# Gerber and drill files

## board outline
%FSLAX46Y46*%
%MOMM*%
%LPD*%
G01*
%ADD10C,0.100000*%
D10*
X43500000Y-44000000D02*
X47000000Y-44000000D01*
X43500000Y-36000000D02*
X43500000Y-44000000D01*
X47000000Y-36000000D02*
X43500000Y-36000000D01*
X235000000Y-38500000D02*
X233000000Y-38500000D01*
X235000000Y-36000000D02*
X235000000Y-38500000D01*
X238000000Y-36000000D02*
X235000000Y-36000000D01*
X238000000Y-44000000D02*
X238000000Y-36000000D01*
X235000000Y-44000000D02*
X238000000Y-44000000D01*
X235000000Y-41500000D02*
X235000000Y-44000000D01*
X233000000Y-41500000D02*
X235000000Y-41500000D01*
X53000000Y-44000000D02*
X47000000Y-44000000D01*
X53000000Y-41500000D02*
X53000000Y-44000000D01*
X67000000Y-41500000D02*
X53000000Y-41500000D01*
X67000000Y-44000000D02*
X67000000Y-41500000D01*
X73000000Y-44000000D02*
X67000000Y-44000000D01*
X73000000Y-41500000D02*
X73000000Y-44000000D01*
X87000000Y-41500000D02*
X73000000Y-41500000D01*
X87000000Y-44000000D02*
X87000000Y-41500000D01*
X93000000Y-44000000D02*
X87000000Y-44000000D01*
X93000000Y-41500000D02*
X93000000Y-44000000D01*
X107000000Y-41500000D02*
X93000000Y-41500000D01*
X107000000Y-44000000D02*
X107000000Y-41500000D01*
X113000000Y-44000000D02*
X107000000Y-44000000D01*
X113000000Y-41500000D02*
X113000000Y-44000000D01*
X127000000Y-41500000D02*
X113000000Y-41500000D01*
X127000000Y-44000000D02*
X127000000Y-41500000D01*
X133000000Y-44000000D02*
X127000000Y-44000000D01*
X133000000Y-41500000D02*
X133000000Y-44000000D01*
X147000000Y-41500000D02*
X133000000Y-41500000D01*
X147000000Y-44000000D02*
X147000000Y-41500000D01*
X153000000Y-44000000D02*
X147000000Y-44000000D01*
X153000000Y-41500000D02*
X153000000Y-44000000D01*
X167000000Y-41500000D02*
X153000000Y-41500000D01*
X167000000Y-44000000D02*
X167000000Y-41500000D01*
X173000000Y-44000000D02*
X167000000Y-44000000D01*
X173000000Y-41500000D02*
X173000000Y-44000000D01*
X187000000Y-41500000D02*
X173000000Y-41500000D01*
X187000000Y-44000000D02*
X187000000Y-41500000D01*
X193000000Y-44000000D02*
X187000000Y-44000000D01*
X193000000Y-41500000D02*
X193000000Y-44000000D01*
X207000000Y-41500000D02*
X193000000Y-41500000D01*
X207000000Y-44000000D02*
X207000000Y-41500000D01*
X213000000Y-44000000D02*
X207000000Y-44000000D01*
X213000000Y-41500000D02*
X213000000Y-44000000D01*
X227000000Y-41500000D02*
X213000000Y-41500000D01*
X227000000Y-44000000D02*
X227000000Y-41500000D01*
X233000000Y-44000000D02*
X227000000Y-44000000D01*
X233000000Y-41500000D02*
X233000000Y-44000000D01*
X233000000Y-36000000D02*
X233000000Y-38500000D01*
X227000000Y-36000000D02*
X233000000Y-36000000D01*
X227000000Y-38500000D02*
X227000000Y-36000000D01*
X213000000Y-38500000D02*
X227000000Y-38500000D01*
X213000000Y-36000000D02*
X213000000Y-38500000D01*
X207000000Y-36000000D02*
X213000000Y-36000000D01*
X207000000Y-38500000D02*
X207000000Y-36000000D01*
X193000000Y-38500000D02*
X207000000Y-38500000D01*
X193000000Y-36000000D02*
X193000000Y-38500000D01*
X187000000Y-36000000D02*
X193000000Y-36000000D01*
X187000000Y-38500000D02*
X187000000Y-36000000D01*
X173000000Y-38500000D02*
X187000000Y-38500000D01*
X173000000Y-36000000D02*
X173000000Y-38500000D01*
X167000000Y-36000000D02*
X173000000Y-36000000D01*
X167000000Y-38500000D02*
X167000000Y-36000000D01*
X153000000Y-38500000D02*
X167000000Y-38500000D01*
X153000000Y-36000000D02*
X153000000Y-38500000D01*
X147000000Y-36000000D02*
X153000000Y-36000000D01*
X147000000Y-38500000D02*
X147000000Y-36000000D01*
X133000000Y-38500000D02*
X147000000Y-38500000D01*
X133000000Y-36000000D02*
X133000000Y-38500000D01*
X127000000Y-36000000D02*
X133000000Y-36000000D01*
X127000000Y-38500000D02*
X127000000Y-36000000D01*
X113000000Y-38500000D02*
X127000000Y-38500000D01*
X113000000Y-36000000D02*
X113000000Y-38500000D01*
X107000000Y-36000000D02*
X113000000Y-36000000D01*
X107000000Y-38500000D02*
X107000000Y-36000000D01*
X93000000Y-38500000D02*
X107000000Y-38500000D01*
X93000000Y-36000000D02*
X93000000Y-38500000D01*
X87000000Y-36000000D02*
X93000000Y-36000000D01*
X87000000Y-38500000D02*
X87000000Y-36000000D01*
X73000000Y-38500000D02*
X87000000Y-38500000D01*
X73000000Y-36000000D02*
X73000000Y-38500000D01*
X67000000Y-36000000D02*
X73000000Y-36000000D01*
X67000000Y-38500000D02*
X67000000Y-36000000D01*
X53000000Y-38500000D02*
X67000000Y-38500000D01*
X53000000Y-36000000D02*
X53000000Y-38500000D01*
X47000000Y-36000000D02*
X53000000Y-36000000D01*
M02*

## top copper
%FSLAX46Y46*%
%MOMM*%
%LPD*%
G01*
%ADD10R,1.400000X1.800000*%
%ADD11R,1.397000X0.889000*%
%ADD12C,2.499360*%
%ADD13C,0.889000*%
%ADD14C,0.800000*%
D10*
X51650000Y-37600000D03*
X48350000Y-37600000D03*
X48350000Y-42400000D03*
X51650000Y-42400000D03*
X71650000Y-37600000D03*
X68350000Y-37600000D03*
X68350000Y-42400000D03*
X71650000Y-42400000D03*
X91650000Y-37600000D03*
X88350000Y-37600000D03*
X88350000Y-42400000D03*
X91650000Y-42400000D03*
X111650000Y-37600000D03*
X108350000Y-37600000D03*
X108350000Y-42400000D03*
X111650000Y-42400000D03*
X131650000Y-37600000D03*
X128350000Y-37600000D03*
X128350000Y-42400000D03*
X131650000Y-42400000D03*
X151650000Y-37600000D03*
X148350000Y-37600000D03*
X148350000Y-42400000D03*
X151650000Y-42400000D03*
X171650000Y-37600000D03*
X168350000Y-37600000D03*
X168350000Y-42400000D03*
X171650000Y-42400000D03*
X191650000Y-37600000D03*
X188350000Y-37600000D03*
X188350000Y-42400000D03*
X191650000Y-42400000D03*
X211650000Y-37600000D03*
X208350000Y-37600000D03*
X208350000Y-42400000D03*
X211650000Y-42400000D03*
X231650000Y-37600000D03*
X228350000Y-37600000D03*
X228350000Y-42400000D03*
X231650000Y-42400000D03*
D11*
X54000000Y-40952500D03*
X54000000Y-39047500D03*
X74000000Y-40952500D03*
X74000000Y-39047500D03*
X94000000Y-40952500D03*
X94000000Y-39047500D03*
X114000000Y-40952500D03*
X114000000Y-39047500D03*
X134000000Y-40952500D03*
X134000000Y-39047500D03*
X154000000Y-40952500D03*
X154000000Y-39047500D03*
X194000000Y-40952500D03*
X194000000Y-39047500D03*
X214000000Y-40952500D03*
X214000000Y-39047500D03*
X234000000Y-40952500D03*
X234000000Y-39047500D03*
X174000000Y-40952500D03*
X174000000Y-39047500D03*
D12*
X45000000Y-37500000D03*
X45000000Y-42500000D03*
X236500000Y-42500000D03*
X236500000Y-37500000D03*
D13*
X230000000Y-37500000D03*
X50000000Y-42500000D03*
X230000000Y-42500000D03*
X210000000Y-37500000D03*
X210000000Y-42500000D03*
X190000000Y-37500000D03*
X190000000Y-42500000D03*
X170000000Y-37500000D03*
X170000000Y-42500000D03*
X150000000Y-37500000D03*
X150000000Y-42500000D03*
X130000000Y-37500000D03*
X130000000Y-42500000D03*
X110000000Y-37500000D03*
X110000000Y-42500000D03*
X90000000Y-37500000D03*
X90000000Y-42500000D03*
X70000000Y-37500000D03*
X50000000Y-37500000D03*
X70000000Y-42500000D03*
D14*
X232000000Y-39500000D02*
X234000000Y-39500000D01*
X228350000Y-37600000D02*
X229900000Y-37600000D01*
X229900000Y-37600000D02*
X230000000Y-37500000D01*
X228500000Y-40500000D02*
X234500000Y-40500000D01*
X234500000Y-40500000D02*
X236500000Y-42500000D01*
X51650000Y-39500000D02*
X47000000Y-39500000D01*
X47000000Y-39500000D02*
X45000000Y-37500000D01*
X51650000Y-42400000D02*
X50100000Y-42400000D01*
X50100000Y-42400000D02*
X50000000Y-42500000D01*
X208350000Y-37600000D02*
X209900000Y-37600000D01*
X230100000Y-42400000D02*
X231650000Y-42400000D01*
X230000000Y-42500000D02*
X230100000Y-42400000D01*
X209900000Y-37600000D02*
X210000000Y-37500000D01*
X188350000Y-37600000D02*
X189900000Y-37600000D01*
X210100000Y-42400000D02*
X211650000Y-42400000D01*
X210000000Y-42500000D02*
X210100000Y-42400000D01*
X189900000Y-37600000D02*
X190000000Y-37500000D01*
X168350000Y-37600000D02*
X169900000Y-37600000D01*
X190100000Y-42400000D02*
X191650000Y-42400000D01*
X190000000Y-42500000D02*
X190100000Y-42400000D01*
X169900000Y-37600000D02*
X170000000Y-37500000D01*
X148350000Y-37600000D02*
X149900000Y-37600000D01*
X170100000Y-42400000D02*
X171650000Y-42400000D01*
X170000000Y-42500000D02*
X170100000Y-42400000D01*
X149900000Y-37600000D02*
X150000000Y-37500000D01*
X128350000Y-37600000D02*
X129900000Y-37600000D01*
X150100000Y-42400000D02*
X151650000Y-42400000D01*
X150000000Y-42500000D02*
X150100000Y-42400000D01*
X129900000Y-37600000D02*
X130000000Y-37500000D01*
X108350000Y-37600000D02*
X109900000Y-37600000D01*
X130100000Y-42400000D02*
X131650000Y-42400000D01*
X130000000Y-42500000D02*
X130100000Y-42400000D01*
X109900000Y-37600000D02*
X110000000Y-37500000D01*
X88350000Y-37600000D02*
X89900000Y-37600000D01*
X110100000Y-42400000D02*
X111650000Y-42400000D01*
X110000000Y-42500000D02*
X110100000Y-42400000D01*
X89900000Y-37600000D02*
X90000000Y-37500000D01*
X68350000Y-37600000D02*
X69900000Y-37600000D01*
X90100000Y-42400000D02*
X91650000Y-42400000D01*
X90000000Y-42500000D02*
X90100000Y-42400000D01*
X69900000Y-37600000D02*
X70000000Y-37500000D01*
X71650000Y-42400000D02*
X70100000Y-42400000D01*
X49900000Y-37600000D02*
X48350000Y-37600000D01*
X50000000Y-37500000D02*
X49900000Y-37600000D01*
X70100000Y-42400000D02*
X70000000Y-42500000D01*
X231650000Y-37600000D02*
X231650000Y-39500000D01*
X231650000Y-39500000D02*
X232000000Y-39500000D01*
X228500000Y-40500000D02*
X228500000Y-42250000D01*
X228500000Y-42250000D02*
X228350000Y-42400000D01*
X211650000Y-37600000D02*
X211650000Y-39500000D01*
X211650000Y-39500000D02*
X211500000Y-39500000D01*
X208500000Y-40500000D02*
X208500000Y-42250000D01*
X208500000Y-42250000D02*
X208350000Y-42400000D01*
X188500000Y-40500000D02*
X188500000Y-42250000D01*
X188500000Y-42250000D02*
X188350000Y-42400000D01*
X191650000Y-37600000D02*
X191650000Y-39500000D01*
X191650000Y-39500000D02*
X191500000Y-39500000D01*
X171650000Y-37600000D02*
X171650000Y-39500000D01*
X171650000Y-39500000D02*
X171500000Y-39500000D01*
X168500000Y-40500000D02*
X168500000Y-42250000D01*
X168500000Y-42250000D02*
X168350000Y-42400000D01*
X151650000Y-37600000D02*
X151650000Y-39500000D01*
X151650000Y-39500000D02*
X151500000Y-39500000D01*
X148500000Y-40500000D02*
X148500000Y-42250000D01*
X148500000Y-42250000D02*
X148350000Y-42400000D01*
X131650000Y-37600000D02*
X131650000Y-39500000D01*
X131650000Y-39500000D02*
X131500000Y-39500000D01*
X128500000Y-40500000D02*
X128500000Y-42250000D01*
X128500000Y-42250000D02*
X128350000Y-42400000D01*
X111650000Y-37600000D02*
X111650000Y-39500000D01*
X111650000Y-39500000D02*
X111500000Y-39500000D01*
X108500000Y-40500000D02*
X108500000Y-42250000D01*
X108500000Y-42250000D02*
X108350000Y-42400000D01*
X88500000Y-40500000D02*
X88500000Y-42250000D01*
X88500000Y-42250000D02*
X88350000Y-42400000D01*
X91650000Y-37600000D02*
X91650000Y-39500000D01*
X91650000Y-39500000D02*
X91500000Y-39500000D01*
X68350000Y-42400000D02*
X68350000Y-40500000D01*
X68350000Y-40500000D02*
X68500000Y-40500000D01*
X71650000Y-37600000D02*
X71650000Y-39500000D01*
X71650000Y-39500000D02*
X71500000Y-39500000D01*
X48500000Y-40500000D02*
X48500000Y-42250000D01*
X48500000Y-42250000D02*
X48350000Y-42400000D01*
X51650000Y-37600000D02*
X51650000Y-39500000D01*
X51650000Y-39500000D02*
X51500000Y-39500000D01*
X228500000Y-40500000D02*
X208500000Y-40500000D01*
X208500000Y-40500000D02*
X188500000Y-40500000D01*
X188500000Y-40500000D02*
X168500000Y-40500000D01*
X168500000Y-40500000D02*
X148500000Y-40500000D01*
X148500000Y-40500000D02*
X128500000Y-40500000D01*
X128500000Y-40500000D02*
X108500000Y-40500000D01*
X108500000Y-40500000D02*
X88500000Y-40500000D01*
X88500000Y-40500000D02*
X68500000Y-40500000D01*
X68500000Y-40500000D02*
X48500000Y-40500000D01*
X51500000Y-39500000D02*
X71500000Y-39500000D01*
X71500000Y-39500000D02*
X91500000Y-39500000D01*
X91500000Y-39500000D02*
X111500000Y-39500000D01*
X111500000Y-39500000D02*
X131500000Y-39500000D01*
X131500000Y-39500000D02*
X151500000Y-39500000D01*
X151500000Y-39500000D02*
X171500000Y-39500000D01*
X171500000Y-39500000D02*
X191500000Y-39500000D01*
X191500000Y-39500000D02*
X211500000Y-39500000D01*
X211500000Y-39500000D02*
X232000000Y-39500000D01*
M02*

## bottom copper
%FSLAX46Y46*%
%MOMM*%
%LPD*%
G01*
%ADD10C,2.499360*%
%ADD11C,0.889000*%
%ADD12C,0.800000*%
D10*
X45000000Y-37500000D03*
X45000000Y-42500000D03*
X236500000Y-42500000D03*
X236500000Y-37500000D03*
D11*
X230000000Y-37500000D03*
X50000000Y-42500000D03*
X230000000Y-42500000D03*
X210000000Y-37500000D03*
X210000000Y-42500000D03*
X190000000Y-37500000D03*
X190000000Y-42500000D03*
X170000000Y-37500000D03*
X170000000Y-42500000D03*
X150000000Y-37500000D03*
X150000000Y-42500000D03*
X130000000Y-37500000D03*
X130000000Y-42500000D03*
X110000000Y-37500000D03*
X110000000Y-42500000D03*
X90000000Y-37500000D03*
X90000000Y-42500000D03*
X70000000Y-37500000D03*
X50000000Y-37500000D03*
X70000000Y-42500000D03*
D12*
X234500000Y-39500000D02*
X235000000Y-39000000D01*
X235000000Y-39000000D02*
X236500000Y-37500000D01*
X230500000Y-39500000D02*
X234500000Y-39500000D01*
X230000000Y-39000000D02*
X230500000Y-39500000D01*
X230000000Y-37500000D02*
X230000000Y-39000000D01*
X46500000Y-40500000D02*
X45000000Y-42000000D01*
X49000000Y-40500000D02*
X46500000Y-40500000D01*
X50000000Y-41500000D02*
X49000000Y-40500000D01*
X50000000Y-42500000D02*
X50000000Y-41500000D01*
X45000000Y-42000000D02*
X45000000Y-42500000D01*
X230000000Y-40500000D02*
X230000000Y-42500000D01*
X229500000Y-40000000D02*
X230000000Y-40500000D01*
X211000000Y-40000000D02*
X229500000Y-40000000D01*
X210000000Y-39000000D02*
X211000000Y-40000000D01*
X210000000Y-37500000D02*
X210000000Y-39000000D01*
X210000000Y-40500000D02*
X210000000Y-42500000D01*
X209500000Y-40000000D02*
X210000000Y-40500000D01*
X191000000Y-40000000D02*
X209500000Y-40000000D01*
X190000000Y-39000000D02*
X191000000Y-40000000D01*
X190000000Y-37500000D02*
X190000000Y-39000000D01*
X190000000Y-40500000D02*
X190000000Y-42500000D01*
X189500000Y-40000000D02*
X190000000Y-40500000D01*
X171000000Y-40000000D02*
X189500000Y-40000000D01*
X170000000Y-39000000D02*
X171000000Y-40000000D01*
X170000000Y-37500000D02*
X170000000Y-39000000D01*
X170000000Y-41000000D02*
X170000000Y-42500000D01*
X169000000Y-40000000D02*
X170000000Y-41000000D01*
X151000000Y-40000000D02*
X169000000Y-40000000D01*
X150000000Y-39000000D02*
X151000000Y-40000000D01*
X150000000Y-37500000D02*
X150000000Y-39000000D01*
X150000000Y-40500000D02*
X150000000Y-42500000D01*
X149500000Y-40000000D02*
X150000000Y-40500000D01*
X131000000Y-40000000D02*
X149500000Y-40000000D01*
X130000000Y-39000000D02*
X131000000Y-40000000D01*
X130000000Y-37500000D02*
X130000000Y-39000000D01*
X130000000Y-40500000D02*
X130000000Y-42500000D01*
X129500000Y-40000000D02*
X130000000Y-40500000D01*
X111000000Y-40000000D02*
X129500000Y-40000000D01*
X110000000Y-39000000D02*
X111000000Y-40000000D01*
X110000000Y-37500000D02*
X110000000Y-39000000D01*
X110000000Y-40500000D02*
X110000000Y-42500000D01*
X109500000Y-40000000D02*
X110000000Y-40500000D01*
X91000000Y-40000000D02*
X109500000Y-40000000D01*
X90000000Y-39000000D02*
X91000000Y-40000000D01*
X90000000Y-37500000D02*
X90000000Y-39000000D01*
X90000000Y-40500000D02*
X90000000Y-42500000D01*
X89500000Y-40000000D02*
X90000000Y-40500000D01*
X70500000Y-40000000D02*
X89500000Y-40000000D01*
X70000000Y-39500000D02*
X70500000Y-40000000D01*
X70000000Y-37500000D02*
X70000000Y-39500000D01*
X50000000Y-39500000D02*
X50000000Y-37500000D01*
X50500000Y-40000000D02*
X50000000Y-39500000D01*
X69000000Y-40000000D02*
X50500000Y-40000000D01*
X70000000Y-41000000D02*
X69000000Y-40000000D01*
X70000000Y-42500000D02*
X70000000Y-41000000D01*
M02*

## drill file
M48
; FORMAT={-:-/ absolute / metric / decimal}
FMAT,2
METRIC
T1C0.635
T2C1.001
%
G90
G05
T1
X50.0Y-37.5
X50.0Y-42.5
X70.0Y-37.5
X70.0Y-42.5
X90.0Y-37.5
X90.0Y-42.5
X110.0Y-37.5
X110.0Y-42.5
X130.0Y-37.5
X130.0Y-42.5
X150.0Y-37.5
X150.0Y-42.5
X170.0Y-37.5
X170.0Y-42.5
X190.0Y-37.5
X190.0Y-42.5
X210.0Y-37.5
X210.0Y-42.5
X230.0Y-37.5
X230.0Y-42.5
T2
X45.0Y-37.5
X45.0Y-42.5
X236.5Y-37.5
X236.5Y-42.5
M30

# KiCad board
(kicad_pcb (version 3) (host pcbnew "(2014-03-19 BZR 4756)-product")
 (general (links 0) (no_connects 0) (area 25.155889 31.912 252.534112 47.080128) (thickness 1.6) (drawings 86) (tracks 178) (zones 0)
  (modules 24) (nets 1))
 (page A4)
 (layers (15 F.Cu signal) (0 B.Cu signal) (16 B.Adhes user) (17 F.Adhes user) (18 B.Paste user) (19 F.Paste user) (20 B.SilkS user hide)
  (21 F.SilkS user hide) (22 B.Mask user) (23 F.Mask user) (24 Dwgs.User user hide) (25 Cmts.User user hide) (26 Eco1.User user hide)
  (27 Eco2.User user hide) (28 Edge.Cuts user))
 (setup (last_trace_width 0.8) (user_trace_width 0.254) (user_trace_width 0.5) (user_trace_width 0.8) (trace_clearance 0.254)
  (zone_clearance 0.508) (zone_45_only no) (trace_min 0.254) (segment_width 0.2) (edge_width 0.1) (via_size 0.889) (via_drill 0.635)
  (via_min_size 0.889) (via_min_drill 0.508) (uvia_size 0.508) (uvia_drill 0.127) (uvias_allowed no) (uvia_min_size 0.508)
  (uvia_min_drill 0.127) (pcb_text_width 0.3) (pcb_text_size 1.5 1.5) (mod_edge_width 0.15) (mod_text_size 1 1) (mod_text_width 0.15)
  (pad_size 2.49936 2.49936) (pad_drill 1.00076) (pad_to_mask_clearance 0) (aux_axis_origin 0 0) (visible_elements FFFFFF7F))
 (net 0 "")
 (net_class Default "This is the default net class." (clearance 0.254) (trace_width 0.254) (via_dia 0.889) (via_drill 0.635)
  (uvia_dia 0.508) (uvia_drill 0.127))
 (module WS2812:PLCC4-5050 (layer F.Cu) (at 50 40)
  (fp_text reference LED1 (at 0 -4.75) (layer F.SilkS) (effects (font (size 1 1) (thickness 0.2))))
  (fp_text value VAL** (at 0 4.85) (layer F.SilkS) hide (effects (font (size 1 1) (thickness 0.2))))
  (pad 1 smd rect (at 1.65 -2.4) (size 1.4 1.8) (layers F.Cu F.Paste F.Mask))
  (pad 2 smd rect (at -1.65 -2.4) (size 1.4 1.8) (layers F.Cu F.Paste F.Mask))
  (pad 3 smd rect (at -1.65 2.4) (size 1.4 1.8) (layers F.Cu F.Paste F.Mask))
  (pad 4 smd rect (at 1.65 2.4) (size 1.4 1.8) (layers F.Cu F.Paste F.Mask)))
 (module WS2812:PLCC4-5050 (layer F.Cu) (at 70 40)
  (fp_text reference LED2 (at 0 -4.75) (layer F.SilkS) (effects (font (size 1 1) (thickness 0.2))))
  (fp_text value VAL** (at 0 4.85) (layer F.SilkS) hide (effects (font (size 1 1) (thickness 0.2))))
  (pad 1 smd rect (at 1.65 -2.4) (size 1.4 1.8) (layers F.Cu F.Paste F.Mask))
  (pad 2 smd rect (at -1.65 -2.4) (size 1.4 1.8) (layers F.Cu F.Paste F.Mask))
  (pad 3 smd rect (at -1.65 2.4) (size 1.4 1.8) (layers F.Cu F.Paste F.Mask))
  (pad 4 smd rect (at 1.65 2.4) (size 1.4 1.8) (layers F.Cu F.Paste F.Mask)))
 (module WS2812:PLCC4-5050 (layer F.Cu) (at 90 40)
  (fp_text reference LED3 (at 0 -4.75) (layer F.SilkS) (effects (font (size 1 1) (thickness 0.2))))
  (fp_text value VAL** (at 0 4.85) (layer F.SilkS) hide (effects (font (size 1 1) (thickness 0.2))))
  (pad 1 smd rect (at 1.65 -2.4) (size 1.4 1.8) (layers F.Cu F.Paste F.Mask))
  (pad 2 smd rect (at -1.65 -2.4) (size 1.4 1.8) (layers F.Cu F.Paste F.Mask))
  (pad 3 smd rect (at -1.65 2.4) (size 1.4 1.8) (layers F.Cu F.Paste F.Mask))
  (pad 4 smd rect (at 1.65 2.4) (size 1.4 1.8) (layers F.Cu F.Paste F.Mask)))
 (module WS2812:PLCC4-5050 (layer F.Cu) (at 110 40)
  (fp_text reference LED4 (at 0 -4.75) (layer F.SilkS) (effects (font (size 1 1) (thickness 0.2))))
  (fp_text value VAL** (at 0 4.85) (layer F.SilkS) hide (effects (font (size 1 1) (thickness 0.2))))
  (pad 1 smd rect (at 1.65 -2.4) (size 1.4 1.8) (layers F.Cu F.Paste F.Mask))
  (pad 2 smd rect (at -1.65 -2.4) (size 1.4 1.8) (layers F.Cu F.Paste F.Mask))
  (pad 3 smd rect (at -1.65 2.4) (size 1.4 1.8) (layers F.Cu F.Paste F.Mask))
  (pad 4 smd rect (at 1.65 2.4) (size 1.4 1.8) (layers F.Cu F.Paste F.Mask)))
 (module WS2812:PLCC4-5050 (layer F.Cu) (at 130 40)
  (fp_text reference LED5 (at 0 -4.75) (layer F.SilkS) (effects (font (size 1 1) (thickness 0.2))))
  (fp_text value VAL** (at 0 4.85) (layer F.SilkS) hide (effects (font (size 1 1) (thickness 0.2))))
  (pad 1 smd rect (at 1.65 -2.4) (size 1.4 1.8) (layers F.Cu F.Paste F.Mask))
  (pad 2 smd rect (at -1.65 -2.4) (size 1.4 1.8) (layers F.Cu F.Paste F.Mask))
  (pad 3 smd rect (at -1.65 2.4) (size 1.4 1.8) (layers F.Cu F.Paste F.Mask))
  (pad 4 smd rect (at 1.65 2.4) (size 1.4 1.8) (layers F.Cu F.Paste F.Mask)))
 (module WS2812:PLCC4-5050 (layer F.Cu) (at 150 40)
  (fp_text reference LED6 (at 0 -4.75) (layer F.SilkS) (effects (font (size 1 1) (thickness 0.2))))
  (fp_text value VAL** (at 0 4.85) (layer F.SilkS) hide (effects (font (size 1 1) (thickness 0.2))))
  (pad 1 smd rect (at 1.65 -2.4) (size 1.4 1.8) (layers F.Cu F.Paste F.Mask))
  (pad 2 smd rect (at -1.65 -2.4) (size 1.4 1.8) (layers F.Cu F.Paste F.Mask))
  (pad 3 smd rect (at -1.65 2.4) (size 1.4 1.8) (layers F.Cu F.Paste F.Mask))
  (pad 4 smd rect (at 1.65 2.4) (size 1.4 1.8) (layers F.Cu F.Paste F.Mask)))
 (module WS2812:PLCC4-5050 (layer F.Cu) (at 170 40)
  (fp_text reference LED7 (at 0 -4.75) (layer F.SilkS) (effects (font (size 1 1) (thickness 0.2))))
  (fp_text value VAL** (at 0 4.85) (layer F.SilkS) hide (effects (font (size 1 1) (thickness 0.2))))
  (pad 1 smd rect (at 1.65 -2.4) (size 1.4 1.8) (layers F.Cu F.Paste F.Mask))
  (pad 2 smd rect (at -1.65 -2.4) (size 1.4 1.8) (layers F.Cu F.Paste F.Mask))
  (pad 3 smd rect (at -1.65 2.4) (size 1.4 1.8) (layers F.Cu F.Paste F.Mask))
  (pad 4 smd rect (at 1.65 2.4) (size 1.4 1.8) (layers F.Cu F.Paste F.Mask)))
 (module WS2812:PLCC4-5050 (layer F.Cu) (at 190 40)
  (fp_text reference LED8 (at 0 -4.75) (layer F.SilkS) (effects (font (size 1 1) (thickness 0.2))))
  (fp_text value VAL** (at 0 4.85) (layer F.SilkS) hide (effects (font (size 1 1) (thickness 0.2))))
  (pad 1 smd rect (at 1.65 -2.4) (size 1.4 1.8) (layers F.Cu F.Paste F.Mask))
  (pad 2 smd rect (at -1.65 -2.4) (size 1.4 1.8) (layers F.Cu F.Paste F.Mask))
  (pad 3 smd rect (at -1.65 2.4) (size 1.4 1.8) (layers F.Cu F.Paste F.Mask))
  (pad 4 smd rect (at 1.65 2.4) (size 1.4 1.8) (layers F.Cu F.Paste F.Mask)))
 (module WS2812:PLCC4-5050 (layer F.Cu) (at 210 40)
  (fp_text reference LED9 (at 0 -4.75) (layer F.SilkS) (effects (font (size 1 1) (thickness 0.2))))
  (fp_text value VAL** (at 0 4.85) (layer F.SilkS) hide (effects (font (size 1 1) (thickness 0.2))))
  (pad 1 smd rect (at 1.65 -2.4) (size 1.4 1.8) (layers F.Cu F.Paste F.Mask))
  (pad 2 smd rect (at -1.65 -2.4) (size 1.4 1.8) (layers F.Cu F.Paste F.Mask))
  (pad 3 smd rect (at -1.65 2.4) (size 1.4 1.8) (layers F.Cu F.Paste F.Mask))
  (pad 4 smd rect (at 1.65 2.4) (size 1.4 1.8) (layers F.Cu F.Paste F.Mask)))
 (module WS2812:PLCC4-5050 (layer F.Cu) (at 230 40)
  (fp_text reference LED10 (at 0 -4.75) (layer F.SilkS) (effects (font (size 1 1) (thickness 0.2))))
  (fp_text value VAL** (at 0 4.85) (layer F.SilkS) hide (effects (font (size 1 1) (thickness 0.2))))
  (pad 1 smd rect (at 1.65 -2.4) (size 1.4 1.8) (layers F.Cu F.Paste F.Mask))
  (pad 2 smd rect (at -1.65 -2.4) (size 1.4 1.8) (layers F.Cu F.Paste F.Mask))
  (pad 3 smd rect (at -1.65 2.4) (size 1.4 1.8) (layers F.Cu F.Paste F.Mask))
  (pad 4 smd rect (at 1.65 2.4) (size 1.4 1.8) (layers F.Cu F.Paste F.Mask)))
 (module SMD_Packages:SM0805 (layer F.Cu) (at 54 40 90)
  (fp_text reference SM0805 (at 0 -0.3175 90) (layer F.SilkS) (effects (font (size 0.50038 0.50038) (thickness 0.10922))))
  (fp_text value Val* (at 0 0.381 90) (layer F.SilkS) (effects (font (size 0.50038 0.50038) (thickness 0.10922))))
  (pad 1 smd rect (at -0.9525 0 90) (size 0.889 1.397) (layers F.Cu F.Paste F.Mask))
  (pad 2 smd rect (at 0.9525 0 90) (size 0.889 1.397) (layers F.Cu F.Paste F.Mask)))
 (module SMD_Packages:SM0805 (layer F.Cu) (at 74 40 90)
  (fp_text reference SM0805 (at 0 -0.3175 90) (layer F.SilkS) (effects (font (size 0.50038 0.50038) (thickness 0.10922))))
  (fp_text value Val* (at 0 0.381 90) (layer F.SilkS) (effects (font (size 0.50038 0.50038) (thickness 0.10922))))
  (pad 1 smd rect (at -0.9525 0 90) (size 0.889 1.397) (layers F.Cu F.Paste F.Mask))
  (pad 2 smd rect (at 0.9525 0 90) (size 0.889 1.397) (layers F.Cu F.Paste F.Mask)))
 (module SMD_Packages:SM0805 (layer F.Cu) (at 94 40 90)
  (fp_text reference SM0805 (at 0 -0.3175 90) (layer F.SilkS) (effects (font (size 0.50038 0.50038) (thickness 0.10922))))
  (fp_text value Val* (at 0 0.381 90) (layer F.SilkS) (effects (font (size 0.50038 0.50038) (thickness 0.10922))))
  (pad 1 smd rect (at -0.9525 0 90) (size 0.889 1.397) (layers F.Cu F.Paste F.Mask))
  (pad 2 smd rect (at 0.9525 0 90) (size 0.889 1.397) (layers F.Cu F.Paste F.Mask)))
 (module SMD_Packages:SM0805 (layer F.Cu) (at 114 40 90)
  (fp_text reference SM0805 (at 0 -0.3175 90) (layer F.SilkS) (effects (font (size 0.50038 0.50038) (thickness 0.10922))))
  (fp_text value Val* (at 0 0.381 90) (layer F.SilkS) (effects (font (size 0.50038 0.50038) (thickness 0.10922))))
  (pad 1 smd rect (at -0.9525 0 90) (size 0.889 1.397) (layers F.Cu F.Paste F.Mask))
  (pad 2 smd rect (at 0.9525 0 90) (size 0.889 1.397) (layers F.Cu F.Paste F.Mask)))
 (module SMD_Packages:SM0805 (layer F.Cu) (at 134 40 90)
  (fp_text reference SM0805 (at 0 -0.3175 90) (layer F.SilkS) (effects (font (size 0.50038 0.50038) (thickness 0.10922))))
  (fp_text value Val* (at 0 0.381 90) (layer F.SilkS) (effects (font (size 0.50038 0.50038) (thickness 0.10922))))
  (pad 1 smd rect (at -0.9525 0 90) (size 0.889 1.397) (layers F.Cu F.Paste F.Mask))
  (pad 2 smd rect (at 0.9525 0 90) (size 0.889 1.397) (layers F.Cu F.Paste F.Mask)))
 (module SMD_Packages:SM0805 (layer F.Cu) (at 154 40 90)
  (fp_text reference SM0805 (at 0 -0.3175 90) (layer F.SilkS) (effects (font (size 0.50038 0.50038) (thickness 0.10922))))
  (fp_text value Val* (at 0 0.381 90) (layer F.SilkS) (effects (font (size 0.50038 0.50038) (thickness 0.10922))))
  (pad 1 smd rect (at -0.9525 0 90) (size 0.889 1.397) (layers F.Cu F.Paste F.Mask))
  (pad 2 smd rect (at 0.9525 0 90) (size 0.889 1.397) (layers F.Cu F.Paste F.Mask)))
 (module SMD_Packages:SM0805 (layer F.Cu) (at 194 40 90)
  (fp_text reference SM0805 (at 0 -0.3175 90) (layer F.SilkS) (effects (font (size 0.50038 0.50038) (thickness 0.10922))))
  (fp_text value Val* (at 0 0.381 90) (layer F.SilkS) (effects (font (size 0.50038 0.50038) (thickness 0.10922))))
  (pad 1 smd rect (at -0.9525 0 90) (size 0.889 1.397) (layers F.Cu F.Paste F.Mask))
  (pad 2 smd rect (at 0.9525 0 90) (size 0.889 1.397) (layers F.Cu F.Paste F.Mask)))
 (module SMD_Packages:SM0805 (layer F.Cu) (at 214 40 90)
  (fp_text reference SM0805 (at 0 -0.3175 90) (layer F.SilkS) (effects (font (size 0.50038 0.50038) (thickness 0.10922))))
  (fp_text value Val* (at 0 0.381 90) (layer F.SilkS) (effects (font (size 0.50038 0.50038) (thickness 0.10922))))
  (pad 1 smd rect (at -0.9525 0 90) (size 0.889 1.397) (layers F.Cu F.Paste F.Mask))
  (pad 2 smd rect (at 0.9525 0 90) (size 0.889 1.397) (layers F.Cu F.Paste F.Mask)))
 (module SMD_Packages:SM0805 (layer F.Cu) (at 234 40 90)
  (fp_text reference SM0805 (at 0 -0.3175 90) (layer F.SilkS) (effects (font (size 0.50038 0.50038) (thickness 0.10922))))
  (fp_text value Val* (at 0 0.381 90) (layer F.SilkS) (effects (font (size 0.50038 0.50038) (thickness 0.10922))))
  (pad 1 smd rect (at -0.9525 0 90) (size 0.889 1.397) (layers F.Cu F.Paste F.Mask))
  (pad 2 smd rect (at 0.9525 0 90) (size 0.889 1.397) (layers F.Cu F.Paste F.Mask)))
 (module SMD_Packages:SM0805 (layer F.Cu) (at 174 40 90)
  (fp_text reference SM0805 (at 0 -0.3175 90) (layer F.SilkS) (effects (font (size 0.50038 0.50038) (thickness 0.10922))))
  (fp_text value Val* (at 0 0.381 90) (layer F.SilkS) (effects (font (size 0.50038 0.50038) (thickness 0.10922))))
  (pad 1 smd rect (at -0.9525 0 90) (size 0.889 1.397) (layers F.Cu F.Paste F.Mask))
  (pad 2 smd rect (at 0.9525 0 90) (size 0.889 1.397) (layers F.Cu F.Paste F.Mask)))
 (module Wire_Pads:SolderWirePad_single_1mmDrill (layer F.Cu) (at 45 37.5)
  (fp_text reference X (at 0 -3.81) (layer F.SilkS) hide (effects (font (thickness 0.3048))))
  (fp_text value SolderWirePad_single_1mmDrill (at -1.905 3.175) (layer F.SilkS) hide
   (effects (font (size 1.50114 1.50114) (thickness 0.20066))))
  (pad 1 thru_hole circle (at 0 0) (size 2.49936 2.49936) (drill 1.00076) (layers *.Cu *.Mask)))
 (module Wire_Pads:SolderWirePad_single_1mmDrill (layer F.Cu) (at 45 42.5)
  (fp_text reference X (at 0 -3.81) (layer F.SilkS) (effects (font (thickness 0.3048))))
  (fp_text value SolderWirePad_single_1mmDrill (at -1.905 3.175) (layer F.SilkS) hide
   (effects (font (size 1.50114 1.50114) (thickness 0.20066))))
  (pad 2 thru_hole circle (at 0 0) (size 2.49936 2.49936) (drill 1.00076) (layers *.Cu *.Mask)))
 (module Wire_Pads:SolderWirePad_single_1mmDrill (layer F.Cu) (at 236.5 42.5)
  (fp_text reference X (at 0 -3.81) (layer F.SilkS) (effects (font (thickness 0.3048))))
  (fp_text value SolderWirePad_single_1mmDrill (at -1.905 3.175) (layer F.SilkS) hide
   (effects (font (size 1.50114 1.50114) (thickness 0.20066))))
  (pad 1 thru_hole circle (at 0 0) (size 2.49936 2.49936) (drill 1.00076) (layers *.Cu *.Mask F.SilkS)))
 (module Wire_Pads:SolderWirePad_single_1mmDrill (layer F.Cu) (at 236.5 37.5)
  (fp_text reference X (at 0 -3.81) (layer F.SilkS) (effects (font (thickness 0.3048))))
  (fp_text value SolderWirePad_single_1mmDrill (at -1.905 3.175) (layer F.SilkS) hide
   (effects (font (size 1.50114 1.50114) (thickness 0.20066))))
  (pad 1 thru_hole circle (at 0 0) (size 2.49936 2.49936) (drill 1.00076) (layers *.Cu *.Mask F.SilkS)))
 (gr_line (start 43.5 44) (end 47 44) (angle 90) (layer Edge.Cuts) (width 0.1))
 (gr_line (start 43.5 36) (end 43.5 44) (angle 90) (layer Edge.Cuts) (width 0.1))
 (gr_line (start 47 36) (end 43.5 36) (angle 90) (layer Edge.Cuts) (width 0.1))
 (gr_line (start 235 38.5) (end 233 38.5) (angle 90) (layer Edge.Cuts) (width 0.1))
 (gr_line (start 235 36) (end 235 38.5) (angle 90) (layer Edge.Cuts) (width 0.1))
 (gr_line (start 238 36) (end 235 36) (angle 90) (layer Edge.Cuts) (width 0.1))
 (gr_line (start 238 44) (end 238 36) (angle 90) (layer Edge.Cuts) (width 0.1))
 (gr_line (start 235 44) (end 238 44) (angle 90) (layer Edge.Cuts) (width 0.1))
 (gr_line (start 235 41.5) (end 235 44) (angle 90) (layer Edge.Cuts) (width 0.1))
 (gr_line (start 233 41.5) (end 235 41.5) (angle 90) (layer Edge.Cuts) (width 0.1))
 (gr_line (start 53 44) (end 47 44) (angle 90) (layer Edge.Cuts) (width 0.1))
 (gr_line (start 53 41.5) (end 53 44) (angle 90) (layer Edge.Cuts) (width 0.1))
 (gr_line (start 67 41.5) (end 53 41.5) (angle 90) (layer Edge.Cuts) (width 0.1))
 (gr_line (start 67 44) (end 67 41.5) (angle 90) (layer Edge.Cuts) (width 0.1))
 (gr_line (start 73 44) (end 67 44) (angle 90) (layer Edge.Cuts) (width 0.1))
 (gr_line (start 73 41.5) (end 73 44) (angle 90) (layer Edge.Cuts) (width 0.1))
 (gr_line (start 87 41.5) (end 73 41.5) (angle 90) (layer Edge.Cuts) (width 0.1))
 (gr_line (start 87 44) (end 87 41.5) (angle 90) (layer Edge.Cuts) (width 0.1))
 (gr_line (start 93 44) (end 87 44) (angle 90) (layer Edge.Cuts) (width 0.1))
 (gr_line (start 93 41.5) (end 93 44) (angle 90) (layer Edge.Cuts) (width 0.1))
 (gr_line (start 107 41.5) (end 93 41.5) (angle 90) (layer Edge.Cuts) (width 0.1))
 (gr_line (start 107 44) (end 107 41.5) (angle 90) (layer Edge.Cuts) (width 0.1))
 (gr_line (start 113 44) (end 107 44) (angle 90) (layer Edge.Cuts) (width 0.1))
 (gr_line (start 113 41.5) (end 113 44) (angle 90) (layer Edge.Cuts) (width 0.1))
 (gr_line (start 127 41.5) (end 113 41.5) (angle 90) (layer Edge.Cuts) (width 0.1))
 (gr_line (start 127 44) (end 127 41.5) (angle 90) (layer Edge.Cuts) (width 0.1))
 (gr_line (start 133 44) (end 127 44) (angle 90) (layer Edge.Cuts) (width 0.1))
 (gr_line (start 133 41.5) (end 133 44) (angle 90) (layer Edge.Cuts) (width 0.1))
 (gr_line (start 147 41.5) (end 133 41.5) (angle 90) (layer Edge.Cuts) (width 0.1))
 (gr_line (start 147 44) (end 147 41.5) (angle 90) (layer Edge.Cuts) (width 0.1))
 (gr_line (start 153 44) (end 147 44) (angle 90) (layer Edge.Cuts) (width 0.1))
 (gr_line (start 153 41.5) (end 153 44) (angle 90) (layer Edge.Cuts) (width 0.1))
 (gr_line (start 167 41.5) (end 153 41.5) (angle 90) (layer Edge.Cuts) (width 0.1))
 (gr_line (start 167 44) (end 167 41.5) (angle 90) (layer Edge.Cuts) (width 0.1))
 (gr_line (start 173 44) (end 167 44) (angle 90) (layer Edge.Cuts) (width 0.1))
 (gr_line (start 173 41.5) (end 173 44) (angle 90) (layer Edge.Cuts) (width 0.1))
 (gr_line (start 187 41.5) (end 173 41.5) (angle 90) (layer Edge.Cuts) (width 0.1))
 (gr_line (start 187 44) (end 187 41.5) (angle 90) (layer Edge.Cuts) (width 0.1))
 (gr_line (start 193 44) (end 187 44) (angle 90) (layer Edge.Cuts) (width 0.1))
 (gr_line (start 193 41.5) (end 193 44) (angle 90) (layer Edge.Cuts) (width 0.1))
 (gr_line (start 207 41.5) (end 193 41.5) (angle 90) (layer Edge.Cuts) (width 0.1))
 (gr_line (start 207 44) (end 207 41.5) (angle 90) (layer Edge.Cuts) (width 0.1))
 (gr_line (start 213 44) (end 207 44) (angle 90) (layer Edge.Cuts) (width 0.1))
 (gr_line (start 213 41.5) (end 213 44) (angle 90) (layer Edge.Cuts) (width 0.1))
 (gr_line (start 227 41.5) (end 213 41.5) (angle 90) (layer Edge.Cuts) (width 0.1))
 (gr_line (start 227 44) (end 227 41.5) (angle 90) (layer Edge.Cuts) (width 0.1))
 (gr_line (start 233 44) (end 227 44) (angle 90) (layer Edge.Cuts) (width 0.1))
 (gr_line (start 233 41.5) (end 233 44) (angle 90) (layer Edge.Cuts) (width 0.1))
 (gr_line (start 233 36) (end 233 38.5) (angle 90) (layer Edge.Cuts) (width 0.1))
 (gr_line (start 227 36) (end 233 36) (angle 90) (layer Edge.Cuts) (width 0.1))
 (gr_line (start 227 38.5) (end 227 36) (angle 90) (layer Edge.Cuts) (width 0.1))
 (gr_line (start 213 38.5) (end 227 38.5) (angle 90) (layer Edge.Cuts) (width 0.1))
 (gr_line (start 213 36) (end 213 38.5) (angle 90) (layer Edge.Cuts) (width 0.1))
 (gr_line (start 207 36) (end 213 36) (angle 90) (layer Edge.Cuts) (width 0.1))
 (gr_line (start 207 38.5) (end 207 36) (angle 90) (layer Edge.Cuts) (width 0.1))
 (gr_line (start 193 38.5) (end 207 38.5) (angle 90) (layer Edge.Cuts) (width 0.1))
 (gr_line (start 193 36) (end 193 38.5) (angle 90) (layer Edge.Cuts) (width 0.1))
 (gr_line (start 187 36) (end 193 36) (angle 90) (layer Edge.Cuts) (width 0.1))
 (gr_line (start 187 38.5) (end 187 36) (angle 90) (layer Edge.Cuts) (width 0.1))
 (gr_line (start 173 38.5) (end 187 38.5) (angle 90) (layer Edge.Cuts) (width 0.1))
 (gr_line (start 173 36) (end 173 38.5) (angle 90) (layer Edge.Cuts) (width 0.1))
 (gr_line (start 167 36) (end 173 36) (angle 90) (layer Edge.Cuts) (width 0.1))
 (gr_line (start 167 38.5) (end 167 36) (angle 90) (layer Edge.Cuts) (width 0.1))
 (gr_line (start 153 38.5) (end 167 38.5) (angle 90) (layer Edge.Cuts) (width 0.1))
 (gr_line (start 153 36) (end 153 38.5) (angle 90) (layer Edge.Cuts) (width 0.1))
 (gr_line (start 147 36) (end 153 36) (angle 90) (layer Edge.Cuts) (width 0.1))
 (gr_line (start 147 38.5) (end 147 36) (angle 90) (layer Edge.Cuts) (width 0.1))
 (gr_line (start 133 38.5) (end 147 38.5) (angle 90) (layer Edge.Cuts) (width 0.1))
 (gr_line (start 133 36) (end 133 38.5) (angle 90) (layer Edge.Cuts) (width 0.1))
 (gr_line (start 127 36) (end 133 36) (angle 90) (layer Edge.Cuts) (width 0.1))
 (gr_line (start 127 38.5) (end 127 36) (angle 90) (layer Edge.Cuts) (width 0.1))
 (gr_line (start 113 38.5) (end 127 38.5) (angle 90) (layer Edge.Cuts) (width 0.1))
 (gr_line (start 113 36) (end 113 38.5) (angle 90) (layer Edge.Cuts) (width 0.1))
 (gr_line (start 107 36) (end 113 36) (angle 90) (layer Edge.Cuts) (width 0.1))
 (gr_line (start 107 38.5) (end 107 36) (angle 90) (layer Edge.Cuts) (width 0.1))
 (gr_line (start 93 38.5) (end 107 38.5) (angle 90) (layer Edge.Cuts) (width 0.1))
 (gr_line (start 93 36) (end 93 38.5) (angle 90) (layer Edge.Cuts) (width 0.1))
 (gr_line (start 87 36) (end 93 36) (angle 90) (layer Edge.Cuts) (width 0.1))
 (gr_line (start 87 38.5) (end 87 36) (angle 90) (layer Edge.Cuts) (width 0.1))
 (gr_line (start 73 38.5) (end 87 38.5) (angle 90) (layer Edge.Cuts) (width 0.1))
 (gr_line (start 73 36) (end 73 38.5) (angle 90) (layer Edge.Cuts) (width 0.1))
 (gr_line (start 67 36) (end 73 36) (angle 90) (layer Edge.Cuts) (width 0.1))
 (gr_line (start 67 38.5) (end 67 36) (angle 90) (layer Edge.Cuts) (width 0.1))
 (gr_line (start 53 38.5) (end 67 38.5) (angle 90) (layer Edge.Cuts) (width 0.1))
 (gr_line (start 53 36) (end 53 38.5) (angle 90) (layer Edge.Cuts) (width 0.1))
 (gr_line (start 47 36) (end 53 36) (angle 90) (layer Edge.Cuts) (width 0.1))
 (segment (start 232 39.5) (end 234 39.5) (width 0.8) (layer F.Cu) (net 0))
 (segment (start 228.35 37.6) (end 229.9 37.6) (width 0.8) (layer F.Cu) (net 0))
 (segment (start 234.5 39.5) (end 235 39) (width 0.8) (layer B.Cu) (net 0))
 (segment (start 235 39) (end 236.5 37.5) (width 0.8) (layer B.Cu) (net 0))
 (segment (start 230.5 39.5) (end 234.5 39.5) (width 0.8) (layer B.Cu) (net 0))
 (segment (start 230 39) (end 230.5 39.5) (width 0.8) (layer B.Cu) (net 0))
 (segment (start 230 37.5) (end 230 39) (width 0.8) (layer B.Cu) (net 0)) (via (at 230 37.5) (size 0.889) (layers F.Cu B.Cu) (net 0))
 (segment (start 229.9 37.6) (end 230 37.5) (width 0.8) (layer F.Cu) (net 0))
 (segment (start 228.5 40.5) (end 234.5 40.5) (width 0.8) (layer F.Cu) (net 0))
 (segment (start 234.5 40.5) (end 236.5 42.5) (width 0.8) (layer F.Cu) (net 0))
 (segment (start 51.65 39.5) (end 47 39.5) (width 0.8) (layer F.Cu) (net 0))
 (segment (start 47 39.5) (end 45 37.5) (width 0.8) (layer F.Cu) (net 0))
 (segment (start 51.65 42.4) (end 50.1 42.4) (width 0.8) (layer F.Cu) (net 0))
 (segment (start 46.5 40.5) (end 45 42) (width 0.8) (layer B.Cu) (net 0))
 (segment (start 49 40.5) (end 46.5 40.5) (width 0.8) (layer B.Cu) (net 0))
 (segment (start 50 41.5) (end 49 40.5) (width 0.8) (layer B.Cu) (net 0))
 (segment (start 50 42.5) (end 50 41.5) (width 0.8) (layer B.Cu) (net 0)) (via (at 50 42.5) (size 0.889) (layers F.Cu B.Cu) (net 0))
 (segment (start 50.1 42.4) (end 50 42.5) (width 0.8) (layer F.Cu) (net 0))
 (segment (start 45 42) (end 45 42.5) (width 0.8) (layer B.Cu) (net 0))
 (segment (start 208.35 37.6) (end 209.9 37.6) (width 0.8) (layer F.Cu) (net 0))
 (segment (start 230.1 42.4) (end 231.65 42.4) (width 0.8) (layer F.Cu) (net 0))
 (segment (start 230 42.5) (end 230.1 42.4) (width 0.8) (layer F.Cu) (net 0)) (via (at 230 42.5) (size 0.889) (layers F.Cu B.Cu) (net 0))
 (segment (start 230 40.5) (end 230 42.5) (width 0.8) (layer B.Cu) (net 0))
 (segment (start 229.5 40) (end 230 40.5) (width 0.8) (layer B.Cu) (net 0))
 (segment (start 211 40) (end 229.5 40) (width 0.8) (layer B.Cu) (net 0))
 (segment (start 210 39) (end 211 40) (width 0.8) (layer B.Cu) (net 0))
 (segment (start 210 37.5) (end 210 39) (width 0.8) (layer B.Cu) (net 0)) (via (at 210 37.5) (size 0.889) (layers F.Cu B.Cu) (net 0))
 (segment (start 209.9 37.6) (end 210 37.5) (width 0.8) (layer F.Cu) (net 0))
 (segment (start 188.35 37.6) (end 189.9 37.6) (width 0.8) (layer F.Cu) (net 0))
 (segment (start 210.1 42.4) (end 211.65 42.4) (width 0.8) (layer F.Cu) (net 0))
 (segment (start 210 42.5) (end 210.1 42.4) (width 0.8) (layer F.Cu) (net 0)) (via (at 210 42.5) (size 0.889) (layers F.Cu B.Cu) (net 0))
 (segment (start 210 40.5) (end 210 42.5) (width 0.8) (layer B.Cu) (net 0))
 (segment (start 209.5 40) (end 210 40.5) (width 0.8) (layer B.Cu) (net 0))
 (segment (start 191 40) (end 209.5 40) (width 0.8) (layer B.Cu) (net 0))
 (segment (start 190 39) (end 191 40) (width 0.8) (layer B.Cu) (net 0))
 (segment (start 190 37.5) (end 190 39) (width 0.8) (layer B.Cu) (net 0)) (via (at 190 37.5) (size 0.889) (layers F.Cu B.Cu) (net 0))
 (segment (start 189.9 37.6) (end 190 37.5) (width 0.8) (layer F.Cu) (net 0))
 (segment (start 168.35 37.6) (end 169.9 37.6) (width 0.8) (layer F.Cu) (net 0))
 (segment (start 190.1 42.4) (end 191.65 42.4) (width 0.8) (layer F.Cu) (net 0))
 (segment (start 190 42.5) (end 190.1 42.4) (width 0.8) (layer F.Cu) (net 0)) (via (at 190 42.5) (size 0.889) (layers F.Cu B.Cu) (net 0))
 (segment (start 190 40.5) (end 190 42.5) (width 0.8) (layer B.Cu) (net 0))
 (segment (start 189.5 40) (end 190 40.5) (width 0.8) (layer B.Cu) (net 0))
 (segment (start 171 40) (end 189.5 40) (width 0.8) (layer B.Cu) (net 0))
 (segment (start 170 39) (end 171 40) (width 0.8) (layer B.Cu) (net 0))
 (segment (start 170 37.5) (end 170 39) (width 0.8) (layer B.Cu) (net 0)) (via (at 170 37.5) (size 0.889) (layers F.Cu B.Cu) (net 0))
 (segment (start 169.9 37.6) (end 170 37.5) (width 0.8) (layer F.Cu) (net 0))
 (segment (start 148.35 37.6) (end 149.9 37.6) (width 0.8) (layer F.Cu) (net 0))
 (segment (start 170.1 42.4) (end 171.65 42.4) (width 0.8) (layer F.Cu) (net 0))
 (segment (start 170 42.5) (end 170.1 42.4) (width 0.8) (layer F.Cu) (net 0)) (via (at 170 42.5) (size 0.889) (layers F.Cu B.Cu) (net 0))
 (segment (start 170 41) (end 170 42.5) (width 0.8) (layer B.Cu) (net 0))
 (segment (start 169 40) (end 170 41) (width 0.8) (layer B.Cu) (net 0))
 (segment (start 151 40) (end 169 40) (width 0.8) (layer B.Cu) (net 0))
 (segment (start 150 39) (end 151 40) (width 0.8) (layer B.Cu) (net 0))
 (segment (start 150 37.5) (end 150 39) (width 0.8) (layer B.Cu) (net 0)) (via (at 150 37.5) (size 0.889) (layers F.Cu B.Cu) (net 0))
 (segment (start 149.9 37.6) (end 150 37.5) (width 0.8) (layer F.Cu) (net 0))
 (segment (start 128.35 37.6) (end 129.9 37.6) (width 0.8) (layer F.Cu) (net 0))
 (segment (start 150.1 42.4) (end 151.65 42.4) (width 0.8) (layer F.Cu) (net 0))
 (segment (start 150 42.5) (end 150.1 42.4) (width 0.8) (layer F.Cu) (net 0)) (via (at 150 42.5) (size 0.889) (layers F.Cu B.Cu) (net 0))
 (segment (start 150 40.5) (end 150 42.5) (width 0.8) (layer B.Cu) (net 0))
 (segment (start 149.5 40) (end 150 40.5) (width 0.8) (layer B.Cu) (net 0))
 (segment (start 131 40) (end 149.5 40) (width 0.8) (layer B.Cu) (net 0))
 (segment (start 130 39) (end 131 40) (width 0.8) (layer B.Cu) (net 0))
 (segment (start 130 37.5) (end 130 39) (width 0.8) (layer B.Cu) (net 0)) (via (at 130 37.5) (size 0.889) (layers F.Cu B.Cu) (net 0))
 (segment (start 129.9 37.6) (end 130 37.5) (width 0.8) (layer F.Cu) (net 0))
 (segment (start 108.35 37.6) (end 109.9 37.6) (width 0.8) (layer F.Cu) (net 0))
 (segment (start 130.1 42.4) (end 131.65 42.4) (width 0.8) (layer F.Cu) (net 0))
 (segment (start 130 42.5) (end 130.1 42.4) (width 0.8) (layer F.Cu) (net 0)) (via (at 130 42.5) (size 0.889) (layers F.Cu B.Cu) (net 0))
 (segment (start 130 40.5) (end 130 42.5) (width 0.8) (layer B.Cu) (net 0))
 (segment (start 129.5 40) (end 130 40.5) (width 0.8) (layer B.Cu) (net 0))
 (segment (start 111 40) (end 129.5 40) (width 0.8) (layer B.Cu) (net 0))
 (segment (start 110 39) (end 111 40) (width 0.8) (layer B.Cu) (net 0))
 (segment (start 110 37.5) (end 110 39) (width 0.8) (layer B.Cu) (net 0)) (via (at 110 37.5) (size 0.889) (layers F.Cu B.Cu) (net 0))
 (segment (start 109.9 37.6) (end 110 37.5) (width 0.8) (layer F.Cu) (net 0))
 (segment (start 88.35 37.6) (end 89.9 37.6) (width 0.8) (layer F.Cu) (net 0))
 (segment (start 110.1 42.4) (end 111.65 42.4) (width 0.8) (layer F.Cu) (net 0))
 (segment (start 110 42.5) (end 110.1 42.4) (width 0.8) (layer F.Cu) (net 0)) (via (at 110 42.5) (size 0.889) (layers F.Cu B.Cu) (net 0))
 (segment (start 110 40.5) (end 110 42.5) (width 0.8) (layer B.Cu) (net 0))
 (segment (start 109.5 40) (end 110 40.5) (width 0.8) (layer B.Cu) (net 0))
 (segment (start 91 40) (end 109.5 40) (width 0.8) (layer B.Cu) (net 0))
 (segment (start 90 39) (end 91 40) (width 0.8) (layer B.Cu) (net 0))
 (segment (start 90 37.5) (end 90 39) (width 0.8) (layer B.Cu) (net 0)) (via (at 90 37.5) (size 0.889) (layers F.Cu B.Cu) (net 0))
 (segment (start 89.9 37.6) (end 90 37.5) (width 0.8) (layer F.Cu) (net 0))
 (segment (start 68.35 37.6) (end 69.9 37.6) (width 0.8) (layer F.Cu) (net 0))
 (segment (start 90.1 42.4) (end 91.65 42.4) (width 0.8) (layer F.Cu) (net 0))
 (segment (start 90 42.5) (end 90.1 42.4) (width 0.8) (layer F.Cu) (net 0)) (via (at 90 42.5) (size 0.889) (layers F.Cu B.Cu) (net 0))
 (segment (start 90 40.5) (end 90 42.5) (width 0.8) (layer B.Cu) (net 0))
 (segment (start 89.5 40) (end 90 40.5) (width 0.8) (layer B.Cu) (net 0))
 (segment (start 70.5 40) (end 89.5 40) (width 0.8) (layer B.Cu) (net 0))
 (segment (start 70 39.5) (end 70.5 40) (width 0.8) (layer B.Cu) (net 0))
 (segment (start 70 37.5) (end 70 39.5) (width 0.8) (layer B.Cu) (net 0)) (via (at 70 37.5) (size 0.889) (layers F.Cu B.Cu) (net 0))
 (segment (start 69.9 37.6) (end 70 37.5) (width 0.8) (layer F.Cu) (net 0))
 (segment (start 71.65 42.4) (end 70.1 42.4) (width 0.8) (layer F.Cu) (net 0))
 (segment (start 49.9 37.6) (end 48.35 37.6) (width 0.8) (layer F.Cu) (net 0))
 (segment (start 50 37.5) (end 49.9 37.6) (width 0.8) (layer F.Cu) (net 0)) (via (at 50 37.5) (size 0.889) (layers F.Cu B.Cu) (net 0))
 (segment (start 50 39.5) (end 50 37.5) (width 0.8) (layer B.Cu) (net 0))
 (segment (start 50.5 40) (end 50 39.5) (width 0.8) (layer B.Cu) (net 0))
 (segment (start 69 40) (end 50.5 40) (width 0.8) (layer B.Cu) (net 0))
 (segment (start 70 41) (end 69 40) (width 0.8) (layer B.Cu) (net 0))
 (segment (start 70 42.5) (end 70 41) (width 0.8) (layer B.Cu) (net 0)) (via (at 70 42.5) (size 0.889) (layers F.Cu B.Cu) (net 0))
 (segment (start 70.1 42.4) (end 70 42.5) (width 0.8) (layer F.Cu) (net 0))
 (segment (start 231.65 37.6) (end 231.65 39.5) (width 0.8) (layer F.Cu) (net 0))
 (segment (start 231.65 39.5) (end 232 39.5) (width 0.8) (layer F.Cu) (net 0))
 (segment (start 228.5 40.5) (end 228.5 42.25) (width 0.8) (layer F.Cu) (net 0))
 (segment (start 228.5 42.25) (end 228.35 42.4) (width 0.8) (layer F.Cu) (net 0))
 (segment (start 211.65 37.6) (end 211.65 39.5) (width 0.8) (layer F.Cu) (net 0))
 (segment (start 211.65 39.5) (end 211.5 39.5) (width 0.8) (layer F.Cu) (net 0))
 (segment (start 208.5 40.5) (end 208.5 42.25) (width 0.8) (layer F.Cu) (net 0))
 (segment (start 208.5 42.25) (end 208.35 42.4) (width 0.8) (layer F.Cu) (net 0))
 (segment (start 188.5 40.5) (end 188.5 42.25) (width 0.8) (layer F.Cu) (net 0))
 (segment (start 188.5 42.25) (end 188.35 42.4) (width 0.8) (layer F.Cu) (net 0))
 (segment (start 191.65 37.6) (end 191.65 39.5) (width 0.8) (layer F.Cu) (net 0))
 (segment (start 191.65 39.5) (end 191.5 39.5) (width 0.8) (layer F.Cu) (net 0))
 (segment (start 171.65 37.6) (end 171.65 39.5) (width 0.8) (layer F.Cu) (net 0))
 (segment (start 171.65 39.5) (end 171.5 39.5) (width 0.8) (layer F.Cu) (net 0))
 (segment (start 168.5 40.5) (end 168.5 42.25) (width 0.8) (layer F.Cu) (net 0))
 (segment (start 168.5 42.25) (end 168.35 42.4) (width 0.8) (layer F.Cu) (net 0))
 (segment (start 151.65 37.6) (end 151.65 39.5) (width 0.8) (layer F.Cu) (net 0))
 (segment (start 151.65 39.5) (end 151.5 39.5) (width 0.8) (layer F.Cu) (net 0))
 (segment (start 148.5 40.5) (end 148.5 42.25) (width 0.8) (layer F.Cu) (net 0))
 (segment (start 148.5 42.25) (end 148.35 42.4) (width 0.8) (layer F.Cu) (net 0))
 (segment (start 131.65 37.6) (end 131.65 39.5) (width 0.8) (layer F.Cu) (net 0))
 (segment (start 131.65 39.5) (end 131.5 39.5) (width 0.8) (layer F.Cu) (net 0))
 (segment (start 128.5 40.5) (end 128.5 42.25) (width 0.8) (layer F.Cu) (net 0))
 (segment (start 128.5 42.25) (end 128.35 42.4) (width 0.8) (layer F.Cu) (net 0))
 (segment (start 111.65 37.6) (end 111.65 39.5) (width 0.8) (layer F.Cu) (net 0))
 (segment (start 111.65 39.5) (end 111.5 39.5) (width 0.8) (layer F.Cu) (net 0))
 (segment (start 108.5 40.5) (end 108.5 42.25) (width 0.8) (layer F.Cu) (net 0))
 (segment (start 108.5 42.25) (end 108.35 42.4) (width 0.8) (layer F.Cu) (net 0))
 (segment (start 88.5 40.5) (end 88.5 42.25) (width 0.8) (layer F.Cu) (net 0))
 (segment (start 88.5 42.25) (end 88.35 42.4) (width 0.8) (layer F.Cu) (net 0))
 (segment (start 91.65 37.6) (end 91.65 39.5) (width 0.8) (layer F.Cu) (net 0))
 (segment (start 91.65 39.5) (end 91.5 39.5) (width 0.8) (layer F.Cu) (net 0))
 (segment (start 68.35 42.4) (end 68.35 40.5) (width 0.8) (layer F.Cu) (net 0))
 (segment (start 68.35 40.5) (end 68.5 40.5) (width 0.8) (layer F.Cu) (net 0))
 (segment (start 71.65 37.6) (end 71.65 39.5) (width 0.8) (layer F.Cu) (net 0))
 (segment (start 71.65 39.5) (end 71.5 39.5) (width 0.8) (layer F.Cu) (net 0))
 (segment (start 48.5 40.5) (end 48.5 42.25) (width 0.8) (layer F.Cu) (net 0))
 (segment (start 48.5 42.25) (end 48.35 42.4) (width 0.8) (layer F.Cu) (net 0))
 (segment (start 51.65 37.6) (end 51.65 39.5) (width 0.8) (layer F.Cu) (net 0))
 (segment (start 51.65 39.5) (end 51.5 39.5) (width 0.8) (layer F.Cu) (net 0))
 (segment (start 228.5 40.5) (end 208.5 40.5) (width 0.8) (layer F.Cu) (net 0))
 (segment (start 208.5 40.5) (end 188.5 40.5) (width 0.8) (layer F.Cu) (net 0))
 (segment (start 188.5 40.5) (end 168.5 40.5) (width 0.8) (layer F.Cu) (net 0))
 (segment (start 168.5 40.5) (end 148.5 40.5) (width 0.8) (layer F.Cu) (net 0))
 (segment (start 148.5 40.5) (end 128.5 40.5) (width 0.8) (layer F.Cu) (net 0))
 (segment (start 128.5 40.5) (end 108.5 40.5) (width 0.8) (layer F.Cu) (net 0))
 (segment (start 108.5 40.5) (end 88.5 40.5) (width 0.8) (layer F.Cu) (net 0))
 (segment (start 88.5 40.5) (end 68.5 40.5) (width 0.8) (layer F.Cu) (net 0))
 (segment (start 68.5 40.5) (end 48.5 40.5) (width 0.8) (layer F.Cu) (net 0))
 (segment (start 51.5 39.5) (end 71.5 39.5) (width 0.8) (layer F.Cu) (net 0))
 (segment (start 71.5 39.5) (end 91.5 39.5) (width 0.8) (layer F.Cu) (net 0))
 (segment (start 91.5 39.5) (end 111.5 39.5) (width 0.8) (layer F.Cu) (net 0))
 (segment (start 111.5 39.5) (end 131.5 39.5) (width 0.8) (layer F.Cu) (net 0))
 (segment (start 131.5 39.5) (end 151.5 39.5) (width 0.8) (layer F.Cu) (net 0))
 (segment (start 151.5 39.5) (end 171.5 39.5) (width 0.8) (layer F.Cu) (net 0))
 (segment (start 171.5 39.5) (end 191.5 39.5) (width 0.8) (layer F.Cu) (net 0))
 (segment (start 191.5 39.5) (end 211.5 39.5) (width 0.8) (layer F.Cu) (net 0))
 (segment (start 211.5 39.5) (end 232 39.5) (width 0.8) (layer F.Cu) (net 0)))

